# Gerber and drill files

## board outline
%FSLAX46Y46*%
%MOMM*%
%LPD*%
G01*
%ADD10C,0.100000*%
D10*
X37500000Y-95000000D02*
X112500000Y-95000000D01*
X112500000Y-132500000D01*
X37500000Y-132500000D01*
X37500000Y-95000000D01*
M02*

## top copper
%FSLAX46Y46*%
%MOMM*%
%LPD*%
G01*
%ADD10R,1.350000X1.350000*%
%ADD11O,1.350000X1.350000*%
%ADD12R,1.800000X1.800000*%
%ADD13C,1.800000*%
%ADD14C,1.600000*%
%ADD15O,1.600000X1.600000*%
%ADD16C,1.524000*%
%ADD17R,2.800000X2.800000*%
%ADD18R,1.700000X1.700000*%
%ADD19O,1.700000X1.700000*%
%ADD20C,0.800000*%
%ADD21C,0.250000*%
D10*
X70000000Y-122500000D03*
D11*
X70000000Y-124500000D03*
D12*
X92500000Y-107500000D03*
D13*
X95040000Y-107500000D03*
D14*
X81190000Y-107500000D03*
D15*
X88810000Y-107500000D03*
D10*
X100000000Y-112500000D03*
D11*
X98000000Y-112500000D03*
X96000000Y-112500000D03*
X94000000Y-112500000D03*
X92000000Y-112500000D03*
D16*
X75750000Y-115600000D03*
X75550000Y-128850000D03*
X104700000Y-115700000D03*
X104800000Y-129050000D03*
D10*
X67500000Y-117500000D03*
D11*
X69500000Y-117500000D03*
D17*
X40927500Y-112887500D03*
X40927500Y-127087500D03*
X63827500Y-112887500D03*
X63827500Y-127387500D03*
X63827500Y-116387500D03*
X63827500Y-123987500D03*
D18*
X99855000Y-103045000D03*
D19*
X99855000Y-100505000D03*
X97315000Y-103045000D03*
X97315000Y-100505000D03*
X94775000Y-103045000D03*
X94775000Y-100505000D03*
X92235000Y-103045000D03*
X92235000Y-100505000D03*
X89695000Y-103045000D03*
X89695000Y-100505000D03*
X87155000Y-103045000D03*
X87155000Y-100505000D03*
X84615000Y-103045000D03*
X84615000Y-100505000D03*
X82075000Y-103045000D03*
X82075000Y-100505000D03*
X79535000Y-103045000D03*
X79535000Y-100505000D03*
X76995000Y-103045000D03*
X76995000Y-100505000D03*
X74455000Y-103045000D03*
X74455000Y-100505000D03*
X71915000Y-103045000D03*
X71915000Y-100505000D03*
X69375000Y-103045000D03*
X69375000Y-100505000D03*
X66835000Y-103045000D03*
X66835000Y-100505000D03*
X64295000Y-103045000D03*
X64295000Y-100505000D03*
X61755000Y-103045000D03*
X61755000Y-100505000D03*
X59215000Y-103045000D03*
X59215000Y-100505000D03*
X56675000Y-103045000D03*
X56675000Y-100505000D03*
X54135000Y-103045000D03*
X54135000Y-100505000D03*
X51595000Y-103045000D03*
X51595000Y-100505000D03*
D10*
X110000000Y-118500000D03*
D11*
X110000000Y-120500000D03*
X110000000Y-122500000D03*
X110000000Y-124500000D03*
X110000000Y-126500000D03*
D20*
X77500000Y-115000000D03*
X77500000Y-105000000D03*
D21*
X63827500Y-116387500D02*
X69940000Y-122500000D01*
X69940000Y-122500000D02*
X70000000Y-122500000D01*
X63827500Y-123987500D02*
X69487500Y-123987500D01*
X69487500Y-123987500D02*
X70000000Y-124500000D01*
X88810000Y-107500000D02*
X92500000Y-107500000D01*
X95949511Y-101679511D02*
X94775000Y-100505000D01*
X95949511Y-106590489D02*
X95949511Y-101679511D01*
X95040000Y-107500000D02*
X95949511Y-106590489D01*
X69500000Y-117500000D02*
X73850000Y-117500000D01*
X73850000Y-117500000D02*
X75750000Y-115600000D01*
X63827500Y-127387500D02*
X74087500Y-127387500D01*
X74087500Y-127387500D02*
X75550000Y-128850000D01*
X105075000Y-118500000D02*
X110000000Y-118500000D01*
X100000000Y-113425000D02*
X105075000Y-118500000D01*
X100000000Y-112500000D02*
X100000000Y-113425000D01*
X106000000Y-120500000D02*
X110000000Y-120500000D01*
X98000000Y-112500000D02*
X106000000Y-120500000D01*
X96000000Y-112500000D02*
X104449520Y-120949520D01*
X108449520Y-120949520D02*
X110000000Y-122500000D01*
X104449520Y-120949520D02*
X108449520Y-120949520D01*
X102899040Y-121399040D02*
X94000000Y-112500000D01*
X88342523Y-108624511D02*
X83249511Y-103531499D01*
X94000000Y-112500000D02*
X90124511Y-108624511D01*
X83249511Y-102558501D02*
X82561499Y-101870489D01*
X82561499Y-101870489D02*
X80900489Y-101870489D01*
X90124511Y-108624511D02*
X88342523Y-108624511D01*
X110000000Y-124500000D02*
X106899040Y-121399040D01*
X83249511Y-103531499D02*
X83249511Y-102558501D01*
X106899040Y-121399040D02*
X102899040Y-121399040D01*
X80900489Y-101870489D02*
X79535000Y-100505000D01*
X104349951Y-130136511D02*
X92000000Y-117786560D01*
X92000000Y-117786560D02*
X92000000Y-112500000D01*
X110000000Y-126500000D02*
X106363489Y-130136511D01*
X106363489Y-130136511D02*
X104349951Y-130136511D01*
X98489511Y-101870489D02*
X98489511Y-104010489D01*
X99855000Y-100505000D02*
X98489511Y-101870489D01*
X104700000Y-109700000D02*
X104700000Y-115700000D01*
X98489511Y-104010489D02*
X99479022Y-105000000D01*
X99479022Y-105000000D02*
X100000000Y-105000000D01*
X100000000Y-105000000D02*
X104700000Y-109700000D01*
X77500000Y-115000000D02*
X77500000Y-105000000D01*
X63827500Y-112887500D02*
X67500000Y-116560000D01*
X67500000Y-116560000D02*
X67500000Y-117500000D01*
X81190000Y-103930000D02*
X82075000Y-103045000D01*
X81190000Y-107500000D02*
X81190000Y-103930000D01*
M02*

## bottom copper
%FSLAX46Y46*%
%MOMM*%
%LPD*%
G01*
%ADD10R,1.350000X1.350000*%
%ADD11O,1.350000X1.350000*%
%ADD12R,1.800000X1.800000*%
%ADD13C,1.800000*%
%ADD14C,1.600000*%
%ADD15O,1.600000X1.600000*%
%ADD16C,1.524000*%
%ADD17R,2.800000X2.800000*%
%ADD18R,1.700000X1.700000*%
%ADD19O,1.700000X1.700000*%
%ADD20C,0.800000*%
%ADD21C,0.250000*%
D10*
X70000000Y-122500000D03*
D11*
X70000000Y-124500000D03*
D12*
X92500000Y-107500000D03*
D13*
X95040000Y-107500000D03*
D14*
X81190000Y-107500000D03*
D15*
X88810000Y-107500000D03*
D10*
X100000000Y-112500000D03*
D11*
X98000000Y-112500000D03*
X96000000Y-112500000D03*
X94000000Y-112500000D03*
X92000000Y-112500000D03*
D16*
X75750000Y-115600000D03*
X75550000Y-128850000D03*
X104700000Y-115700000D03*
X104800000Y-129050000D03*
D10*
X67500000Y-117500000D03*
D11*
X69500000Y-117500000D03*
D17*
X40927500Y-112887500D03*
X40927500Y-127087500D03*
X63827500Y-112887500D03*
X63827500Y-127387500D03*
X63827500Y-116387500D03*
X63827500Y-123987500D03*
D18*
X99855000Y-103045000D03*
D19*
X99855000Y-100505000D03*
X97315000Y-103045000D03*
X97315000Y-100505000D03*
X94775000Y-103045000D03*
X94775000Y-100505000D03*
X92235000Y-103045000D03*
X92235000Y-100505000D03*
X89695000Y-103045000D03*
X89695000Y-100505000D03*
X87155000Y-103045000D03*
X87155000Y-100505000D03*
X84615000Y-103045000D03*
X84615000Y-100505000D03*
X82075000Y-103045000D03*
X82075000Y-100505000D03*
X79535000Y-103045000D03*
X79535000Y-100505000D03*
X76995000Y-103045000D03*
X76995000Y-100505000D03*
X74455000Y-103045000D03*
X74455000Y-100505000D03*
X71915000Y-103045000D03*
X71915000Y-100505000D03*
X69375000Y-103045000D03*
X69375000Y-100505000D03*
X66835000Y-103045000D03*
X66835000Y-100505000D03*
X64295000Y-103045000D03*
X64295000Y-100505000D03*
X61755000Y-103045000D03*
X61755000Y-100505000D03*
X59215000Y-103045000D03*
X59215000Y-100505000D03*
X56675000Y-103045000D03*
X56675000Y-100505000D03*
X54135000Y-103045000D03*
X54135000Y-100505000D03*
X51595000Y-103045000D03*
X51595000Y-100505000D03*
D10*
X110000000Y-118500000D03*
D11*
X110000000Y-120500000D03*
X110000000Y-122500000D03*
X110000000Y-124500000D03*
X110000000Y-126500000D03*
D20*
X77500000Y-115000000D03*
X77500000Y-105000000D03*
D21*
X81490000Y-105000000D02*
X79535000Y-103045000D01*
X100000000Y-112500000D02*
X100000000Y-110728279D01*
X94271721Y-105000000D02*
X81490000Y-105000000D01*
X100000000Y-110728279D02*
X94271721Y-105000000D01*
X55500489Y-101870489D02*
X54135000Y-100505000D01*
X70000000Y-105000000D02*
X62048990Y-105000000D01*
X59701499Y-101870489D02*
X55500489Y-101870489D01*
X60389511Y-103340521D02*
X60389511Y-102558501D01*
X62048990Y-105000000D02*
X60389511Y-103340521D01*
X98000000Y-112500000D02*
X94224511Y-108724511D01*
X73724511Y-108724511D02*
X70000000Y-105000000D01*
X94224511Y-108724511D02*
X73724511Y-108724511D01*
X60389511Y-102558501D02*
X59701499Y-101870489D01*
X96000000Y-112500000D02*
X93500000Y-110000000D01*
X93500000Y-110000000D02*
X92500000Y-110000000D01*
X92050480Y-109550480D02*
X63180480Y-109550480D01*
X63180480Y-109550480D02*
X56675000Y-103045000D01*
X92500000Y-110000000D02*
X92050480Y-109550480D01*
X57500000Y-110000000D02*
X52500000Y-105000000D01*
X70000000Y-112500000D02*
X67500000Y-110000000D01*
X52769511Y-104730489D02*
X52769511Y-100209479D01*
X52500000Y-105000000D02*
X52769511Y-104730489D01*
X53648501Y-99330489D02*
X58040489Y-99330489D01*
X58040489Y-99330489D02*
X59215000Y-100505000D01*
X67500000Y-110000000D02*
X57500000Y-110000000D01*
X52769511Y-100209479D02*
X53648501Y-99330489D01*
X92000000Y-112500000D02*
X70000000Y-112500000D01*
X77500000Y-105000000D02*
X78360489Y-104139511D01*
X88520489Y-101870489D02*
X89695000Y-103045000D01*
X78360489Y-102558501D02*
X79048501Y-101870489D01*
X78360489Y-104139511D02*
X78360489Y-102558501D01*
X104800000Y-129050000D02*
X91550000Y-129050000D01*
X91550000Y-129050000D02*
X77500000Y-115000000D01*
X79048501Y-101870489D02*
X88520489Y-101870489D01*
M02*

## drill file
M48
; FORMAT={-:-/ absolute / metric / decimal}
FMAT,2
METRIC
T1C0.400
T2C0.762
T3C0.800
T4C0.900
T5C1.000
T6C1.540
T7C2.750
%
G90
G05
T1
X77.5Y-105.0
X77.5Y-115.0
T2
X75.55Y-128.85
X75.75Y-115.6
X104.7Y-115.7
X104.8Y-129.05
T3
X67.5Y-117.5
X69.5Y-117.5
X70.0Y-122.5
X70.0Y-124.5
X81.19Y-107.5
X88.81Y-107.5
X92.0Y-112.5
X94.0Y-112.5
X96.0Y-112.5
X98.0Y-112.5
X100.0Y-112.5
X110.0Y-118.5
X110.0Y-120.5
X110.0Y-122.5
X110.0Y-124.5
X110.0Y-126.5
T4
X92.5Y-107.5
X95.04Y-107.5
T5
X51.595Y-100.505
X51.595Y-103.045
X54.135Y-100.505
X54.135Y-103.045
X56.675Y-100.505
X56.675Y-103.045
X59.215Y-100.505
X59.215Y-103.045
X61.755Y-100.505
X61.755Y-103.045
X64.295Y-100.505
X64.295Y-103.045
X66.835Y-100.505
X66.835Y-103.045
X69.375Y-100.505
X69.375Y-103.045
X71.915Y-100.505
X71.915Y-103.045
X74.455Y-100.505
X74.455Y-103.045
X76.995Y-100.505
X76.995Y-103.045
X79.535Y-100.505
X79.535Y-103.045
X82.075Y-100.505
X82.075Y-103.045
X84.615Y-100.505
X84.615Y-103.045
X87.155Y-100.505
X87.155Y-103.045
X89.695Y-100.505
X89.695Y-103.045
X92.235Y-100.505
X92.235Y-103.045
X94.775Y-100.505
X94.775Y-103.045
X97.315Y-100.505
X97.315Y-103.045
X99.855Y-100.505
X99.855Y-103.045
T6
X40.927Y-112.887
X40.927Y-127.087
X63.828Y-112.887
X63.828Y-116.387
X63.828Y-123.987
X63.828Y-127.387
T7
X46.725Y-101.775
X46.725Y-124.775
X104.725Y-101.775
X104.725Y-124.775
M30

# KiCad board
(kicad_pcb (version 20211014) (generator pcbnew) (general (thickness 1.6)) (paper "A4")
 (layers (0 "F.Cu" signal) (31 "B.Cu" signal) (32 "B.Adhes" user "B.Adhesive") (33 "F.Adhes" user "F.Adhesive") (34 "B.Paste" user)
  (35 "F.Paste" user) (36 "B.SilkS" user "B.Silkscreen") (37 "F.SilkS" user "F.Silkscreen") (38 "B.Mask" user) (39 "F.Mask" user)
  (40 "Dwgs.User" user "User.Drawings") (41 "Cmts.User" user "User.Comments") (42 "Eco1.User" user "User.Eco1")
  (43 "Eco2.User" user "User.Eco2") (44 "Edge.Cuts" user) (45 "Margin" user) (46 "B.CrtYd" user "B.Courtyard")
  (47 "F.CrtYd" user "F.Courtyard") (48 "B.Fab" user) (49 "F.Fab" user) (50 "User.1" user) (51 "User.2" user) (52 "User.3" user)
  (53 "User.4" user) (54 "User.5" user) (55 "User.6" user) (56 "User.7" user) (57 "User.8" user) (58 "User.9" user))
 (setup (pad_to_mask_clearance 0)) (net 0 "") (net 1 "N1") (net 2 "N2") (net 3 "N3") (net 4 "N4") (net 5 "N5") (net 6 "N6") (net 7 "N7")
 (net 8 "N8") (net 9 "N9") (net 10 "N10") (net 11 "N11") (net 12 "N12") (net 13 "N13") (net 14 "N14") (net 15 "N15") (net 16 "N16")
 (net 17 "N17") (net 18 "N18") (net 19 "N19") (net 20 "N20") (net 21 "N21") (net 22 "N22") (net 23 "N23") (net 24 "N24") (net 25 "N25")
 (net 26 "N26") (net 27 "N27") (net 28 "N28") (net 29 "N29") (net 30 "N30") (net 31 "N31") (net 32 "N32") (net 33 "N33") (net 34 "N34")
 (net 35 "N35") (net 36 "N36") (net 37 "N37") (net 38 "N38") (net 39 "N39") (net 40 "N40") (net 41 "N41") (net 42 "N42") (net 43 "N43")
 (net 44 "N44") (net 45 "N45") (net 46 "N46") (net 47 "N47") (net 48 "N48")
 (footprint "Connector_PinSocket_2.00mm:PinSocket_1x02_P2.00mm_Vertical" (layer "F.Cu") (at 70 122.5)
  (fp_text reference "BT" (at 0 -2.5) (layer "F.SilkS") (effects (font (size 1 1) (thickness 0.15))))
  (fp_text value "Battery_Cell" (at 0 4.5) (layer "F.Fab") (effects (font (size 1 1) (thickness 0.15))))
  (pad "1" thru_hole rect (at 0 0) (size 1.35 1.35) (drill 0.8) (layers *.Cu *.Mask) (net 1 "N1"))
  (pad "2" thru_hole oval (at 0 2) (size 1.35 1.35) (drill 0.8) (layers *.Cu *.Mask) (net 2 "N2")))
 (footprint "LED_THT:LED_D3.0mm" (layer "F.Cu") (at 92.5 107.5)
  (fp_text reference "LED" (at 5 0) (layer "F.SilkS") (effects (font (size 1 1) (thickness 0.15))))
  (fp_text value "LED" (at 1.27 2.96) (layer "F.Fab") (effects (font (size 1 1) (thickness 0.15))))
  (pad "1" thru_hole rect (at 0 0) (size 1.8 1.8) (drill 0.9) (layers *.Cu *.Mask) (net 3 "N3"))
  (pad "2" thru_hole circle (at 2.54 0) (size 1.8 1.8) (drill 0.9) (layers *.Cu *.Mask) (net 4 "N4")))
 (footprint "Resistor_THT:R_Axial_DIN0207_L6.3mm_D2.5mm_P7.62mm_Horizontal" (layer "F.Cu") (at 81.19 107.5)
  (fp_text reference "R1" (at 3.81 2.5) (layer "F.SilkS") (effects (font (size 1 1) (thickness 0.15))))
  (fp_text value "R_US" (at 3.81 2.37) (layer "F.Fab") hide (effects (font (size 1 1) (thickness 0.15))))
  (pad "1" thru_hole circle (at 0 0) (size 1.6 1.6) (drill 0.8) (layers *.Cu *.Mask) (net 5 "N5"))
  (pad "2" thru_hole oval (at 7.62 0) (size 1.6 1.6) (drill 0.8) (layers *.Cu *.Mask) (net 3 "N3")))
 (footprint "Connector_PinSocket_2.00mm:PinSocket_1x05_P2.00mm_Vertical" (layer "F.Cu") (at 100 112.5 -90)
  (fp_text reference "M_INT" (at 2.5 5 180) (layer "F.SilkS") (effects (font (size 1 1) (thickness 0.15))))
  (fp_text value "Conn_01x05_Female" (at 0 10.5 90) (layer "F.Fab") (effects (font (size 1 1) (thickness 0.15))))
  (pad "1" thru_hole rect (at 0 0 270) (size 1.35 1.35) (drill 0.8) (layers *.Cu *.Mask) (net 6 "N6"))
  (pad "2" thru_hole oval (at 0 2 270) (size 1.35 1.35) (drill 0.8) (layers *.Cu *.Mask) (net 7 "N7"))
  (pad "3" thru_hole oval (at 0 4 270) (size 1.35 1.35) (drill 0.8) (layers *.Cu *.Mask) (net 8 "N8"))
  (pad "4" thru_hole oval (at 0 6 270) (size 1.35 1.35) (drill 0.8) (layers *.Cu *.Mask) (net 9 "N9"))
  (pad "5" thru_hole oval (at 0 8 270) (size 1.35 1.35) (drill 0.8) (layers *.Cu *.Mask) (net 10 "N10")))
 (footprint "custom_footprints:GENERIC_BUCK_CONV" (layer "F.Cu") (at 90 122.5)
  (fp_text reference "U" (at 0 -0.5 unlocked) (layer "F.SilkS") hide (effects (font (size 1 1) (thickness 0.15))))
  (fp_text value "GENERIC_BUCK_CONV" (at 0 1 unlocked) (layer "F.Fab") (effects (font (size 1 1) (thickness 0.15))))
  (pad "1" thru_hole circle (at -14.25 -6.9) (size 1.524 1.524) (drill 0.762) (layers *.Cu *.Mask) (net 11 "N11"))
  (pad "2" thru_hole circle (at -14.45 6.35) (size 1.524 1.524) (drill 0.762) (layers *.Cu *.Mask) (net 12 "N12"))
  (pad "3" thru_hole circle (at 14.7 -6.8) (size 1.524 1.524) (drill 0.762) (layers *.Cu *.Mask) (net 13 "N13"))
  (pad "4" thru_hole circle (at 14.8 6.55) (size 1.524 1.524) (drill 0.762) (layers *.Cu *.Mask) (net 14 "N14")))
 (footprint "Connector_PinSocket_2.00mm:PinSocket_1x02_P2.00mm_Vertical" (layer "F.Cu") (at 67.5 117.5 90)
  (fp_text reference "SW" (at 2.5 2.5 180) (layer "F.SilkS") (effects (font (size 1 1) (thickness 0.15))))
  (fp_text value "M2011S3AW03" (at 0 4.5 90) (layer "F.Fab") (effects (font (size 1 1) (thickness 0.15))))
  (pad "1" thru_hole rect (at 0 0 90) (size 1.35 1.35) (drill 0.8) (layers *.Cu *.Mask) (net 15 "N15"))
  (pad "2" thru_hole oval (at 0 2 90) (size 1.35 1.35) (drill 0.8) (layers *.Cu *.Mask) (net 11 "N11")))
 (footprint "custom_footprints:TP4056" (layer "F.Cu") (at 39.2275 111.1875)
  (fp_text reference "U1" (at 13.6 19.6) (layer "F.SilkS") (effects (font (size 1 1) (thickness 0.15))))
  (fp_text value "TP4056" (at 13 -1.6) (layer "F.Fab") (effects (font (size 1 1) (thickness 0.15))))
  (pad "1" thru_hole rect (at 1.7 1.7) (size 2.8 2.8) (drill 1.54) (layers *.Cu *.Mask) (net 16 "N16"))
  (pad "2" thru_hole rect (at 1.7 15.9) (size 2.8 2.8) (drill 1.54) (layers *.Cu *.Mask) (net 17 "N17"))
  (pad "3" thru_hole rect (at 24.6 1.7) (size 2.8 2.8) (drill 1.54) (layers *.Cu *.Mask) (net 15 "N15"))
  (pad "4" thru_hole rect (at 24.6 16.2) (size 2.8 2.8) (drill 1.54) (layers *.Cu *.Mask) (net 12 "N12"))
  (pad "5" thru_hole rect (at 24.6 5.2) (size 2.8 2.8) (drill 1.54) (layers *.Cu *.Mask) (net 1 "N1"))
  (pad "6" thru_hole rect (at 24.6 12.8) (size 2.8 2.8) (drill 1.54) (layers *.Cu *.Mask) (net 2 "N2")))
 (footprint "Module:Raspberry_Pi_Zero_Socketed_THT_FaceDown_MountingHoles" (layer "F.Cu") (at 99.855 103.045 -90)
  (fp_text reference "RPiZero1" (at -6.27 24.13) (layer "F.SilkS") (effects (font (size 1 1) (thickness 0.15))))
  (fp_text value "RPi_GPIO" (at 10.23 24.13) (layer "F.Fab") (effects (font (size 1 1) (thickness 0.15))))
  (pad "" np_thru_hole circle (at 21.73 -4.87) (size 2.75 2.75) (drill 2.75) (layers *.Cu *.Mask) (solder_mask_margin 1.625))
  (pad "" np_thru_hole circle (at -1.27 53.13) (size 2.75 2.75) (drill 2.75) (layers *.Cu *.Mask) (solder_mask_margin 1.625))
  (pad "" np_thru_hole circle (at -1.27 -4.87) (size 2.75 2.75) (drill 2.75) (layers *.Cu *.Mask) (solder_mask_margin 1.625))
  (pad "" np_thru_hole circle (at 21.73 53.13) (size 2.75 2.75) (drill 2.75) (layers *.Cu *.Mask) (solder_mask_margin 1.625))
  (pad "1" thru_hole rect (at 0 0 270) (size 1.7 1.7) (drill 1) (layers *.Cu *.Mask) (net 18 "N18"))
  (pad "2" thru_hole oval (at -2.54 0 270) (size 1.7 1.7) (drill 1) (layers *.Cu *.Mask) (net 13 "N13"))
  (pad "3" thru_hole oval (at 0 2.54 270) (size 1.7 1.7) (drill 1) (layers *.Cu *.Mask) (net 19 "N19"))
  (pad "4" thru_hole oval (at -2.54 2.54 270) (size 1.7 1.7) (drill 1) (layers *.Cu *.Mask) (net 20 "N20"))
  (pad "5" thru_hole oval (at 0 5.08 270) (size 1.7 1.7) (drill 1) (layers *.Cu *.Mask) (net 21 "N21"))
  (pad "6" thru_hole oval (at -2.54 5.08 270) (size 1.7 1.7) (drill 1) (layers *.Cu *.Mask) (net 4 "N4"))
  (pad "7" thru_hole oval (at 0 7.62 270) (size 1.7 1.7) (drill 1) (layers *.Cu *.Mask) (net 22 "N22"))
  (pad "8" thru_hole oval (at -2.54 7.62 270) (size 1.7 1.7) (drill 1) (layers *.Cu *.Mask) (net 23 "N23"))
  (pad "9" thru_hole oval (at 0 10.16 270) (size 1.7 1.7) (drill 1) (layers *.Cu *.Mask) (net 14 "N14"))
  (pad "10" thru_hole oval (at -2.54 10.16 270) (size 1.7 1.7) (drill 1) (layers *.Cu *.Mask) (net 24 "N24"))
  (pad "11" thru_hole oval (at 0 12.7 270) (size 1.7 1.7) (drill 1) (layers *.Cu *.Mask) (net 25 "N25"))
  (pad "12" thru_hole oval (at -2.54 12.7 270) (size 1.7 1.7) (drill 1) (layers *.Cu *.Mask) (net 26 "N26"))
  (pad "13" thru_hole oval (at 0 15.24 270) (size 1.7 1.7) (drill 1) (layers *.Cu *.Mask) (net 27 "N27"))
  (pad "14" thru_hole oval (at -2.54 15.24 270) (size 1.7 1.7) (drill 1) (layers *.Cu *.Mask) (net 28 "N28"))
  (pad "15" thru_hole oval (at 0 17.78 270) (size 1.7 1.7) (drill 1) (layers *.Cu *.Mask) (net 5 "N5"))
  (pad "16" thru_hole oval (at -2.54 17.78 270) (size 1.7 1.7) (drill 1) (layers *.Cu *.Mask) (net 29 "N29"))
  (pad "17" thru_hole oval (at 0 20.32 270) (size 1.7 1.7) (drill 1) (layers *.Cu *.Mask) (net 6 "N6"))
  (pad "18" thru_hole oval (at -2.54 20.32 270) (size 1.7 1.7) (drill 1) (layers *.Cu *.Mask) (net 9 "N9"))
  (pad "19" thru_hole oval (at 0 22.86 270) (size 1.7 1.7) (drill 1) (layers *.Cu *.Mask) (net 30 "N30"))
  (pad "20" thru_hole oval (at -2.54 22.86 270) (size 1.7 1.7) (drill 1) (layers *.Cu *.Mask) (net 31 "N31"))
  (pad "21" thru_hole oval (at 0 25.4 270) (size 1.7 1.7) (drill 1) (layers *.Cu *.Mask) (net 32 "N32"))
  (pad "22" thru_hole oval (at -2.54 25.4 270) (size 1.7 1.7) (drill 1) (layers *.Cu *.Mask) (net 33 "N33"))
  (pad "23" thru_hole oval (at 0 27.94 270) (size 1.7 1.7) (drill 1) (layers *.Cu *.Mask) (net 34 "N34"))
  (pad "24" thru_hole oval (at -2.54 27.94 270) (size 1.7 1.7) (drill 1) (layers *.Cu *.Mask) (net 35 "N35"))
  (pad "25" thru_hole oval (at 0 30.48 270) (size 1.7 1.7) (drill 1) (layers *.Cu *.Mask) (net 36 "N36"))
  (pad "26" thru_hole oval (at -2.54 30.48 270) (size 1.7 1.7) (drill 1) (layers *.Cu *.Mask) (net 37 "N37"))
  (pad "27" thru_hole oval (at 0 33.02 270) (size 1.7 1.7) (drill 1) (layers *.Cu *.Mask) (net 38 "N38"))
  (pad "28" thru_hole oval (at -2.54 33.02 270) (size 1.7 1.7) (drill 1) (layers *.Cu *.Mask) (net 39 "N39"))
  (pad "29" thru_hole oval (at 0 35.56 270) (size 1.7 1.7) (drill 1) (layers *.Cu *.Mask) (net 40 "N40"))
  (pad "30" thru_hole oval (at -2.54 35.56 270) (size 1.7 1.7) (drill 1) (layers *.Cu *.Mask) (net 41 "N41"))
  (pad "31" thru_hole oval (at 0 38.1 270) (size 1.7 1.7) (drill 1) (layers *.Cu *.Mask) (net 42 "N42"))
  (pad "32" thru_hole oval (at -2.54 38.1 270) (size 1.7 1.7) (drill 1) (layers *.Cu *.Mask) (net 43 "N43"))
  (pad "33" thru_hole oval (at 0 40.64 270) (size 1.7 1.7) (drill 1) (layers *.Cu *.Mask) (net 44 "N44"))
  (pad "34" thru_hole oval (at -2.54 40.64 270) (size 1.7 1.7) (drill 1) (layers *.Cu *.Mask) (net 10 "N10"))
  (pad "35" thru_hole oval (at 0 43.18 270) (size 1.7 1.7) (drill 1) (layers *.Cu *.Mask) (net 8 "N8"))
  (pad "36" thru_hole oval (at -2.54 43.18 270) (size 1.7 1.7) (drill 1) (layers *.Cu *.Mask) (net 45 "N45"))
  (pad "37" thru_hole oval (at 0 45.72 270) (size 1.7 1.7) (drill 1) (layers *.Cu *.Mask) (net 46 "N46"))
  (pad "38" thru_hole oval (at -2.54 45.72 270) (size 1.7 1.7) (drill 1) (layers *.Cu *.Mask) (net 7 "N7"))
  (pad "39" thru_hole oval (at 0 48.26 270) (size 1.7 1.7) (drill 1) (layers *.Cu *.Mask) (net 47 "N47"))
  (pad "40" thru_hole oval (at -2.54 48.26 270) (size 1.7 1.7) (drill 1) (layers *.Cu *.Mask) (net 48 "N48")))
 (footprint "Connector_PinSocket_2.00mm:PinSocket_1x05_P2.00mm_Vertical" (layer "F.Cu") (at 110 118.5)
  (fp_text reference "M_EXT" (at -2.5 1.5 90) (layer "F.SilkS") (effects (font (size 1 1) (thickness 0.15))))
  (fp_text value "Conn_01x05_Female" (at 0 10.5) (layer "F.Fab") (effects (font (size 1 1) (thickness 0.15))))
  (pad "1" thru_hole rect (at 0 0) (size 1.35 1.35) (drill 0.8) (layers *.Cu *.Mask) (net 6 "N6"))
  (pad "2" thru_hole oval (at 0 2) (size 1.35 1.35) (drill 0.8) (layers *.Cu *.Mask) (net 7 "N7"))
  (pad "3" thru_hole oval (at 0 4) (size 1.35 1.35) (drill 0.8) (layers *.Cu *.Mask) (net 8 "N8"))
  (pad "4" thru_hole oval (at 0 6) (size 1.35 1.35) (drill 0.8) (layers *.Cu *.Mask) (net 9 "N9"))
  (pad "5" thru_hole oval (at 0 8) (size 1.35 1.35) (drill 0.8) (layers *.Cu *.Mask) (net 10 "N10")))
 (gr_rect (start 37.5 95) (end 112.5 132.5) (layer "Edge.Cuts") (width 0.1) (fill none))
 (segment (start 63.8275 116.3875) (end 69.94 122.5) (width 0.25) (layer "F.Cu") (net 1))
 (segment (start 69.94 122.5) (end 70 122.5) (width 0.25) (layer "F.Cu") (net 1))
 (segment (start 63.8275 123.9875) (end 69.4875 123.9875) (width 0.25) (layer "F.Cu") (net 2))
 (segment (start 69.4875 123.9875) (end 70 124.5) (width 0.25) (layer "F.Cu") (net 2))
 (segment (start 88.81 107.5) (end 92.5 107.5) (width 0.25) (layer "F.Cu") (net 3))
 (segment (start 95.949511 101.679511) (end 94.775 100.505) (width 0.25) (layer "F.Cu") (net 4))
 (segment (start 95.949511 106.590489) (end 95.949511 101.679511) (width 0.25) (layer "F.Cu") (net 4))
 (segment (start 95.04 107.5) (end 95.949511 106.590489) (width 0.25) (layer "F.Cu") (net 4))
 (segment (start 69.5 117.5) (end 73.85 117.5) (width 0.25) (layer "F.Cu") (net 11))
 (segment (start 73.85 117.5) (end 75.75 115.6) (width 0.25) (layer "F.Cu") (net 11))
 (segment (start 63.8275 127.3875) (end 74.0875 127.3875) (width 0.25) (layer "F.Cu") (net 12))
 (segment (start 74.0875 127.3875) (end 75.55 128.85) (width 0.25) (layer "F.Cu") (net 12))
 (segment (start 105.075 118.5) (end 110 118.5) (width 0.25) (layer "F.Cu") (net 6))
 (segment (start 100 113.425) (end 105.075 118.5) (width 0.25) (layer "F.Cu") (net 6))
 (segment (start 100 112.5) (end 100 113.425) (width 0.25) (layer "F.Cu") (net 6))
 (segment (start 81.49 105) (end 79.535 103.045) (width 0.25) (layer "B.Cu") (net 6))
 (segment (start 100 112.5) (end 100 110.728279) (width 0.25) (layer "B.Cu") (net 6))
 (segment (start 94.271721 105) (end 81.49 105) (width 0.25) (layer "B.Cu") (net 6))
 (segment (start 100 110.728279) (end 94.271721 105) (width 0.25) (layer "B.Cu") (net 6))
 (segment (start 106 120.5) (end 110 120.5) (width 0.25) (layer "F.Cu") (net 7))
 (segment (start 98 112.5) (end 106 120.5) (width 0.25) (layer "F.Cu") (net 7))
 (segment (start 55.500489 101.870489) (end 54.135 100.505) (width 0.25) (layer "B.Cu") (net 7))
 (segment (start 70 105) (end 62.04899 105) (width 0.25) (layer "B.Cu") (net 7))
 (segment (start 59.701499 101.870489) (end 55.500489 101.870489) (width 0.25) (layer "B.Cu") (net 7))
 (segment (start 60.389511 103.340521) (end 60.389511 102.558501) (width 0.25) (layer "B.Cu") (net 7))
 (segment (start 62.04899 105) (end 60.389511 103.340521) (width 0.25) (layer "B.Cu") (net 7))
 (segment (start 98 112.5) (end 94.224511 108.724511) (width 0.25) (layer "B.Cu") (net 7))
 (segment (start 73.724511 108.724511) (end 70 105) (width 0.25) (layer "B.Cu") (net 7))
 (segment (start 94.224511 108.724511) (end 73.724511 108.724511) (width 0.25) (layer "B.Cu") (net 7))
 (segment (start 60.389511 102.558501) (end 59.701499 101.870489) (width 0.25) (layer "B.Cu") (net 7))
 (segment (start 96 112.5) (end 104.44952 120.94952) (width 0.25) (layer "F.Cu") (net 8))
 (segment (start 108.44952 120.94952) (end 110 122.5) (width 0.25) (layer "F.Cu") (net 8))
 (segment (start 104.44952 120.94952) (end 108.44952 120.94952) (width 0.25) (layer "F.Cu") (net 8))
 (segment (start 96 112.5) (end 93.5 110) (width 0.25) (layer "B.Cu") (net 8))
 (segment (start 93.5 110) (end 92.5 110) (width 0.25) (layer "B.Cu") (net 8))
 (segment (start 92.05048 109.55048) (end 63.18048 109.55048) (width 0.25) (layer "B.Cu") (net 8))
 (segment (start 63.18048 109.55048) (end 56.675 103.045) (width 0.25) (layer "B.Cu") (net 8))
 (segment (start 92.5 110) (end 92.05048 109.55048) (width 0.25) (layer "B.Cu") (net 8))
 (segment (start 102.89904 121.39904) (end 94 112.5) (width 0.25) (layer "F.Cu") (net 9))
 (segment (start 88.342523 108.624511) (end 83.249511 103.531499) (width 0.25) (layer "F.Cu") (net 9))
 (segment (start 94 112.5) (end 90.124511 108.624511) (width 0.25) (layer "F.Cu") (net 9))
 (segment (start 83.249511 102.558501) (end 82.561499 101.870489) (width 0.25) (layer "F.Cu") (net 9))
 (segment (start 82.561499 101.870489) (end 80.900489 101.870489) (width 0.25) (layer "F.Cu") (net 9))
 (segment (start 90.124511 108.624511) (end 88.342523 108.624511) (width 0.25) (layer "F.Cu") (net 9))
 (segment (start 110 124.5) (end 106.89904 121.39904) (width 0.25) (layer "F.Cu") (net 9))
 (segment (start 83.249511 103.531499) (end 83.249511 102.558501) (width 0.25) (layer "F.Cu") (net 9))
 (segment (start 106.89904 121.39904) (end 102.89904 121.39904) (width 0.25) (layer "F.Cu") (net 9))
 (segment (start 80.900489 101.870489) (end 79.535 100.505) (width 0.25) (layer "F.Cu") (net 9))
 (segment (start 104.349951 130.136511) (end 92 117.78656) (width 0.25) (layer "F.Cu") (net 10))
 (segment (start 92 117.78656) (end 92 112.5) (width 0.25) (layer "F.Cu") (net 10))
 (segment (start 110 126.5) (end 106.363489 130.136511) (width 0.25) (layer "F.Cu") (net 10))
 (segment (start 106.363489 130.136511) (end 104.349951 130.136511) (width 0.25) (layer "F.Cu") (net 10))
 (segment (start 57.5 110) (end 52.5 105) (width 0.25) (layer "B.Cu") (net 10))
 (segment (start 70 112.5) (end 67.5 110) (width 0.25) (layer "B.Cu") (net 10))
 (segment (start 52.769511 104.730489) (end 52.769511 100.209479) (width 0.25) (layer "B.Cu") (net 10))
 (segment (start 52.5 105) (end 52.769511 104.730489) (width 0.25) (layer "B.Cu") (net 10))
 (segment (start 53.648501 99.330489) (end 58.040489 99.330489) (width 0.25) (layer "B.Cu") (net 10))
 (segment (start 58.040489 99.330489) (end 59.215 100.505) (width 0.25) (layer "B.Cu") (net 10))
 (segment (start 67.5 110) (end 57.5 110) (width 0.25) (layer "B.Cu") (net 10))
 (segment (start 52.769511 100.209479) (end 53.648501 99.330489) (width 0.25) (layer "B.Cu") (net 10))
 (segment (start 92 112.5) (end 70 112.5) (width 0.25) (layer "B.Cu") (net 10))
 (segment (start 98.489511 101.870489) (end 98.489511 104.010489) (width 0.25) (layer "F.Cu") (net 13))
 (segment (start 99.855 100.505) (end 98.489511 101.870489) (width 0.25) (layer "F.Cu") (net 13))
 (segment (start 104.7 109.7) (end 104.7 115.7) (width 0.25) (layer "F.Cu") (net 13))
 (segment (start 98.489511 104.010489) (end 99.479022 105) (width 0.25) (layer "F.Cu") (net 13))
 (segment (start 99.479022 105) (end 100 105) (width 0.25) (layer "F.Cu") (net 13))
 (segment (start 100 105) (end 104.7 109.7) (width 0.25) (layer "F.Cu") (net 13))
 (segment (start 77.5 115) (end 77.5 105) (width 0.25) (layer "F.Cu") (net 14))
 (via (at 77.5 115) (size 0.8) (drill 0.4) (layers "F.Cu" "B.Cu") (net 14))
 (via (at 77.5 105) (size 0.8) (drill 0.4) (layers "F.Cu" "B.Cu") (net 14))
 (segment (start 77.5 105) (end 78.360489 104.139511) (width 0.25) (layer "B.Cu") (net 14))
 (segment (start 88.520489 101.870489) (end 89.695 103.045) (width 0.25) (layer "B.Cu") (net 14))
 (segment (start 78.360489 102.558501) (end 79.048501 101.870489) (width 0.25) (layer "B.Cu") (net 14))
 (segment (start 78.360489 104.139511) (end 78.360489 102.558501) (width 0.25) (layer "B.Cu") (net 14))
 (segment (start 104.8 129.05) (end 91.55 129.05) (width 0.25) (layer "B.Cu") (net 14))
 (segment (start 91.55 129.05) (end 77.5 115) (width 0.25) (layer "B.Cu") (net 14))
 (segment (start 79.048501 101.870489) (end 88.520489 101.870489) (width 0.25) (layer "B.Cu") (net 14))
 (segment (start 63.8275 112.8875) (end 67.5 116.56) (width 0.25) (layer "F.Cu") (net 15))
 (segment (start 67.5 116.56) (end 67.5 117.5) (width 0.25) (layer "F.Cu") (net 15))
 (segment (start 81.19 103.93) (end 82.075 103.045) (width 0.25) (layer "F.Cu") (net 5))
 (segment (start 81.19 107.5) (end 81.19 103.93) (width 0.25) (layer "F.Cu") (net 5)))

